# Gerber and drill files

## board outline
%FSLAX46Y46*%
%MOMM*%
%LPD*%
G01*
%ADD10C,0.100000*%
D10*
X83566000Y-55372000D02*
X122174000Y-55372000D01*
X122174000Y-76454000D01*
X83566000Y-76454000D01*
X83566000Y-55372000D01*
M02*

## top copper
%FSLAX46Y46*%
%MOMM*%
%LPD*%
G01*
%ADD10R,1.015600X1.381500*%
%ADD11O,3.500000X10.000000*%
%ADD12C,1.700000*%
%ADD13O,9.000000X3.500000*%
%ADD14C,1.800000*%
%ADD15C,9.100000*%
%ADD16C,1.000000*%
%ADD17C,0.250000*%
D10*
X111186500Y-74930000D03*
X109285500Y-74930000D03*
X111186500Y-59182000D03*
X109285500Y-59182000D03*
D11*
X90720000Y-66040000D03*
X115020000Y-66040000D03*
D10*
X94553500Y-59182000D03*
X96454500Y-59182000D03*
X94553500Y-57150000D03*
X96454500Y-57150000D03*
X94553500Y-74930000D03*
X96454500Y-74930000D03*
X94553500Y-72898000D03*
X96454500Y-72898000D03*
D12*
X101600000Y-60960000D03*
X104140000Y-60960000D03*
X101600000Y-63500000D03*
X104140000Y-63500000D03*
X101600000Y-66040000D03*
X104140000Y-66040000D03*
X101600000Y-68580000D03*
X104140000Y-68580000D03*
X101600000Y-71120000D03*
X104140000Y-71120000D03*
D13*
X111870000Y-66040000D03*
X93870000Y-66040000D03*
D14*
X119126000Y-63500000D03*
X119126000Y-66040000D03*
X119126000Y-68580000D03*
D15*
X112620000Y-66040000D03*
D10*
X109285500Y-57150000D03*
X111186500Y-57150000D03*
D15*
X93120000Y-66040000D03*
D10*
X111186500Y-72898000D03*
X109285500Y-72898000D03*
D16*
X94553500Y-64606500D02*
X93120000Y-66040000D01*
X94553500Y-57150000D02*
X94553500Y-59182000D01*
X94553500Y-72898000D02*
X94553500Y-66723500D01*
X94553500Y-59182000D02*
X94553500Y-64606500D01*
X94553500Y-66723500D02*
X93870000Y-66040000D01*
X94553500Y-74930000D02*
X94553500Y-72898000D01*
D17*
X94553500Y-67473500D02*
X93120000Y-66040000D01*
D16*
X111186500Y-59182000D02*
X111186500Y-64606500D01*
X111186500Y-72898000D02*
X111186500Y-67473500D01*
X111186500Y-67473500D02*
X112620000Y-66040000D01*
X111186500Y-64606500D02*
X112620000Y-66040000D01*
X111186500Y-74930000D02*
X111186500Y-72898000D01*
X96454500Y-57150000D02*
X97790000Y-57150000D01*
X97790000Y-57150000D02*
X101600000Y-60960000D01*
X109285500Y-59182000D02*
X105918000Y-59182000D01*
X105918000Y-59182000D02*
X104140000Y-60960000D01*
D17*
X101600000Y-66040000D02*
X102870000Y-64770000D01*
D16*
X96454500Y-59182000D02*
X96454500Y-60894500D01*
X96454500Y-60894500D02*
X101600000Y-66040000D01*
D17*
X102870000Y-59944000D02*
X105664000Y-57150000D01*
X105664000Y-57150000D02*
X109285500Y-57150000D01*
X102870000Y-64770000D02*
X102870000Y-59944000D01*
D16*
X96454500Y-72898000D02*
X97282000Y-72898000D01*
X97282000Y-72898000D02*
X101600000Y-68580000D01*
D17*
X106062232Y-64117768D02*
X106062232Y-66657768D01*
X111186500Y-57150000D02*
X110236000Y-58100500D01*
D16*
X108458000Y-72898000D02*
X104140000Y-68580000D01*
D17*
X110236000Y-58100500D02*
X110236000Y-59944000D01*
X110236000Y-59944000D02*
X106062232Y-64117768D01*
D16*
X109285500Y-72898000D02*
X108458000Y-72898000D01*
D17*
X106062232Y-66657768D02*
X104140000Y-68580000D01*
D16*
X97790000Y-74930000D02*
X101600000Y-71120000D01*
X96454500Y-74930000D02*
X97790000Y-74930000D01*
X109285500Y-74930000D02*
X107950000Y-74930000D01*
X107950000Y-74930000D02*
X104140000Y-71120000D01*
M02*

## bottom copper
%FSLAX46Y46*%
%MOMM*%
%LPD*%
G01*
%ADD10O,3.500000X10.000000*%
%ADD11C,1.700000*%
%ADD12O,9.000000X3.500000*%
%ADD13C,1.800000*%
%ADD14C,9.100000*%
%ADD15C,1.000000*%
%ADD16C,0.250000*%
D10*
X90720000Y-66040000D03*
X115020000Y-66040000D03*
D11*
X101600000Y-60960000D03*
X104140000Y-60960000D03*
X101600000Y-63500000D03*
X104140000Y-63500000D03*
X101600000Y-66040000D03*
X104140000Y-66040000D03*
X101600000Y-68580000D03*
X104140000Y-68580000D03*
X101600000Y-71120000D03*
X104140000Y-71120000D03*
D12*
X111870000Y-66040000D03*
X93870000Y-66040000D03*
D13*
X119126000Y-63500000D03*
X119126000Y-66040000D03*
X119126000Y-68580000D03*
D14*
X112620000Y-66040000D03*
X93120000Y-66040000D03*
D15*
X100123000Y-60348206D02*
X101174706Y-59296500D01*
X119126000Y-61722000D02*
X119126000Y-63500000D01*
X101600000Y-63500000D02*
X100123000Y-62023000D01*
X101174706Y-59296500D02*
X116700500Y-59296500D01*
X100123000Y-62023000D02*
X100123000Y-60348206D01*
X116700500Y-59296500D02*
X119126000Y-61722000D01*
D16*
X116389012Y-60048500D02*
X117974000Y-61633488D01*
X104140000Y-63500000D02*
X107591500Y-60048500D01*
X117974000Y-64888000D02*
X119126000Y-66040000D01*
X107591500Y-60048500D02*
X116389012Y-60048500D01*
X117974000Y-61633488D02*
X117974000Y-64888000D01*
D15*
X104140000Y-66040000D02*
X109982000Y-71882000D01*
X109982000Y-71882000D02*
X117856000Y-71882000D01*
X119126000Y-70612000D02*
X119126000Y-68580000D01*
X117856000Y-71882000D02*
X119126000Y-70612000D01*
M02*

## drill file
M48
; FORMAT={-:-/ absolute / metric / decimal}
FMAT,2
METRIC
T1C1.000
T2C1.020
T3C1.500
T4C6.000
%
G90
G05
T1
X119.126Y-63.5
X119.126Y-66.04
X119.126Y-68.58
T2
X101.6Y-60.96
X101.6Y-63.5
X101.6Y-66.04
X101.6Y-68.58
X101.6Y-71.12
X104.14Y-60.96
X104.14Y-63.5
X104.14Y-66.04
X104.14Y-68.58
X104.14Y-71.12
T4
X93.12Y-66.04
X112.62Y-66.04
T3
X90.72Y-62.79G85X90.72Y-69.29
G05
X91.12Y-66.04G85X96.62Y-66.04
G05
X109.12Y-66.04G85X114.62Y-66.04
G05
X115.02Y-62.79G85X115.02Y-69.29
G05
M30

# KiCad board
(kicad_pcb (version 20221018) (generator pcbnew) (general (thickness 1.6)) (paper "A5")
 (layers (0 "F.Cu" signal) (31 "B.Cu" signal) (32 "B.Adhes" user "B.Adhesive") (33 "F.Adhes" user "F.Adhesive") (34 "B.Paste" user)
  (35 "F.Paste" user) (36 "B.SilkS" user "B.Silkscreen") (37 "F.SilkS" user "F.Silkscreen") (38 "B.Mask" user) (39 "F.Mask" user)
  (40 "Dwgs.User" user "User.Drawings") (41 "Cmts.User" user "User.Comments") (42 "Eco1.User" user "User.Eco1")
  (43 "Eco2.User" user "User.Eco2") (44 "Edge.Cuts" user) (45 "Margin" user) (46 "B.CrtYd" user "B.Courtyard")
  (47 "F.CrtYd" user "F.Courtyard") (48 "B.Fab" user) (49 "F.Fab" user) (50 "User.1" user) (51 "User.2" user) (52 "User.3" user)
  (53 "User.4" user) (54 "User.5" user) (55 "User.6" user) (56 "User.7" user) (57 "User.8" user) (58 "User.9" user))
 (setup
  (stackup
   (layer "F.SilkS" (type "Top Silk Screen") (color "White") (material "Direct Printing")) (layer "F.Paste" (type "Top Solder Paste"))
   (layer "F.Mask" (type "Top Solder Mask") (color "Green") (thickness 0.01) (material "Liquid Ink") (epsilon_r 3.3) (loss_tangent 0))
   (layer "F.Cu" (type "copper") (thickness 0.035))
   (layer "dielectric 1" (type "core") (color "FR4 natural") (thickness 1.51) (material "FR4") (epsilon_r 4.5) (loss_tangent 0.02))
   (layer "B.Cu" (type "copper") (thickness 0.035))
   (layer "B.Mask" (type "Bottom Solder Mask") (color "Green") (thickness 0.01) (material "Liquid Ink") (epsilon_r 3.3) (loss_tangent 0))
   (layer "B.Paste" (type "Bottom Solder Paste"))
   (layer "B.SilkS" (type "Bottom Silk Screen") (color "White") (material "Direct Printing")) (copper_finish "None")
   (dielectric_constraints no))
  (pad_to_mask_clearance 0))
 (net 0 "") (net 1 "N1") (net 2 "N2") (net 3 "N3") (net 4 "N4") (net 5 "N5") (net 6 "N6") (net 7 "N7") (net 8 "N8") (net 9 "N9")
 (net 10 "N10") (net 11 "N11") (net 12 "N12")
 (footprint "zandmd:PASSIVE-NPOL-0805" (layer "F.Cu") (at 110.236 74.93 180)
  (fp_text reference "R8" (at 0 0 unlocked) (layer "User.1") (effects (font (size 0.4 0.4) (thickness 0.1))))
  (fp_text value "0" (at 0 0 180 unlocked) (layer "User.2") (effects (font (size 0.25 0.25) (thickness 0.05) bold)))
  (pad "1" smd rect (at -0.9505 0 180) (size 1.0156 1.3815) (layers "F.Cu" "F.Paste" "F.Mask") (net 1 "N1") (thermal_bridge_angle 45))
  (pad "2" smd rect (at 0.9505 0 180) (size 1.0156 1.3815) (layers "F.Cu" "F.Paste" "F.Mask") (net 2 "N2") (thermal_bridge_angle 45)))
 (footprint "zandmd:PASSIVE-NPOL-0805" (layer "F.Cu") (at 110.236 59.182 180)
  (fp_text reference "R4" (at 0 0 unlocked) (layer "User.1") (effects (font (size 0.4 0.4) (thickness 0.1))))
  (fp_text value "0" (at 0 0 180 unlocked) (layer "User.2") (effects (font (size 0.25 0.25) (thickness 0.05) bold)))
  (pad "1" smd rect (at -0.9505 0 180) (size 1.0156 1.3815) (layers "F.Cu" "F.Paste" "F.Mask") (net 1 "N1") (thermal_bridge_angle 45))
  (pad "2" smd rect (at 0.9505 0 180) (size 1.0156 1.3815) (layers "F.Cu" "F.Paste" "F.Mask") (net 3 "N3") (thermal_bridge_angle 45)))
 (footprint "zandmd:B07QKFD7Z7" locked (layer "F.Cu") (at 102.87 66.04) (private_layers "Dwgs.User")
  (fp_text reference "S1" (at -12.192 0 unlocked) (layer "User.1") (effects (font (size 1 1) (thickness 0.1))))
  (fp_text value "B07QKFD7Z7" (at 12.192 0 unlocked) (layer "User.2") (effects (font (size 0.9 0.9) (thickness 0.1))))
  (pad "1" thru_hole oval locked (at -12.15 0) (size 3.5 10) (drill oval 1.5 8) (layers "*.Cu" "*.Mask") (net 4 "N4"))
  (pad "2" thru_hole oval locked (at 12.15 0) (size 3.5 10) (drill oval 1.5 8) (layers "*.Cu" "*.Mask") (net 1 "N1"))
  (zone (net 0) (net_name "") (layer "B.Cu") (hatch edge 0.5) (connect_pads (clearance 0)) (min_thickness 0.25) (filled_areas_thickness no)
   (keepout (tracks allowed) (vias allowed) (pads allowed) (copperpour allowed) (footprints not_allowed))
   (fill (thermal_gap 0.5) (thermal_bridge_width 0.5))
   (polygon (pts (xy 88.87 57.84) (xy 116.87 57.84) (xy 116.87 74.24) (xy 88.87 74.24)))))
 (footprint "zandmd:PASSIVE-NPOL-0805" (layer "F.Cu") (at 95.504 59.182)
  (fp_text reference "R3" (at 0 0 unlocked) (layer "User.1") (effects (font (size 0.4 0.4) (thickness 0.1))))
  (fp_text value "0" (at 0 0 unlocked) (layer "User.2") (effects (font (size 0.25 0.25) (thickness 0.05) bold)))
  (pad "1" smd rect (at -0.9505 0) (size 1.0156 1.3815) (layers "F.Cu" "F.Paste" "F.Mask") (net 4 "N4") (thermal_bridge_angle 45))
  (pad "2" smd rect (at 0.9505 0) (size 1.0156 1.3815) (layers "F.Cu" "F.Paste" "F.Mask") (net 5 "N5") (thermal_bridge_angle 45)))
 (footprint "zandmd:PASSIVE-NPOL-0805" (layer "F.Cu") (at 95.504 57.15)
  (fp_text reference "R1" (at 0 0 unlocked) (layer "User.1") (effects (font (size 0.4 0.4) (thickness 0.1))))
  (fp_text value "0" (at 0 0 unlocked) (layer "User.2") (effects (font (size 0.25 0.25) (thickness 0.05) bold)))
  (pad "1" smd rect (at -0.9505 0) (size 1.0156 1.3815) (layers "F.Cu" "F.Paste" "F.Mask") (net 4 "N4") (thermal_bridge_angle 45))
  (pad "2" smd rect (at 0.9505 0) (size 1.0156 1.3815) (layers "F.Cu" "F.Paste" "F.Mask") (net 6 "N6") (thermal_bridge_angle 45)))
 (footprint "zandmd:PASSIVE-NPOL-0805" (layer "F.Cu") (at 95.504 74.93)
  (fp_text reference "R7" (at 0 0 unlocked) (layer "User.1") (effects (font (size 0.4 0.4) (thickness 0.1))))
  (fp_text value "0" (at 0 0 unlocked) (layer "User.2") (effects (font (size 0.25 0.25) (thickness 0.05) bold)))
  (pad "1" smd rect (at -0.9505 0) (size 1.0156 1.3815) (layers "F.Cu" "F.Paste" "F.Mask") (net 4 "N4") (thermal_bridge_angle 45))
  (pad "2" smd rect (at 0.9505 0) (size 1.0156 1.3815) (layers "F.Cu" "F.Paste" "F.Mask") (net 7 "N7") (thermal_bridge_angle 45)))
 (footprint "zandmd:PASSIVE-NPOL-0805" (layer "F.Cu") (at 95.504 72.898)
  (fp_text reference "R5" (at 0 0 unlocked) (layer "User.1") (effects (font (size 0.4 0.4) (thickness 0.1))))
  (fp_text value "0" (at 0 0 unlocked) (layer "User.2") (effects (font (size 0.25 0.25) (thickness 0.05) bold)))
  (pad "1" smd rect (at -0.9505 0) (size 1.0156 1.3815) (layers "F.Cu" "F.Paste" "F.Mask") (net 4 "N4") (thermal_bridge_angle 45))
  (pad "2" smd rect (at 0.9505 0) (size 1.0156 1.3815) (layers "F.Cu" "F.Paste" "F.Mask") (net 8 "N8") (thermal_bridge_angle 45)))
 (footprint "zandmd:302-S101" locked (layer "F.Cu") (at 102.87 66.04 -90)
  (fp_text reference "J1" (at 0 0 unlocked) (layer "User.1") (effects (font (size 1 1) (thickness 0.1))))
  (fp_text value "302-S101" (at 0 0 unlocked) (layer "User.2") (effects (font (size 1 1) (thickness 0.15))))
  (pad "1" thru_hole circle locked (at -5.08 1.27 270) (size 1.7 1.7) (drill 1.02) (layers "*.Cu" "*.Mask") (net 6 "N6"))
  (pad "2" thru_hole circle locked (at -5.08 -1.27 270) (size 1.7 1.7) (drill 1.02) (layers "*.Cu" "*.Mask") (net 3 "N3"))
  (pad "3" thru_hole circle locked (at -2.54 1.27 270) (size 1.7 1.7) (drill 1.02) (layers "*.Cu" "*.Mask") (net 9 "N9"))
  (pad "4" thru_hole circle locked (at -2.54 -1.27 270) (size 1.7 1.7) (drill 1.02) (layers "*.Cu" "*.Mask") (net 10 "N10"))
  (pad "5" thru_hole circle locked (at 0 1.27 270) (size 1.7 1.7) (drill 1.02) (layers "*.Cu" "*.Mask") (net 5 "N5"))
  (pad "6" thru_hole circle locked (at 0 -1.27 270) (size 1.7 1.7) (drill 1.02) (layers "*.Cu" "*.Mask") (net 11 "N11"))
  (pad "7" thru_hole circle locked (at 2.54 1.27 270) (size 1.7 1.7) (drill 1.02) (layers "*.Cu" "*.Mask") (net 8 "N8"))
  (pad "8" thru_hole circle locked (at 2.54 -1.27 270) (size 1.7 1.7) (drill 1.02) (layers "*.Cu" "*.Mask") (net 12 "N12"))
  (pad "9" thru_hole circle locked (at 5.08 1.27 270) (size 1.7 1.7) (drill 1.02) (layers "*.Cu" "*.Mask") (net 7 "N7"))
  (pad "10" thru_hole circle locked (at 5.08 -1.27 270) (size 1.7 1.7) (drill 1.02) (layers "*.Cu" "*.Mask") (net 2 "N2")))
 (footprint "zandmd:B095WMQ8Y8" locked (layer "F.Cu") (at 102.87 66.04) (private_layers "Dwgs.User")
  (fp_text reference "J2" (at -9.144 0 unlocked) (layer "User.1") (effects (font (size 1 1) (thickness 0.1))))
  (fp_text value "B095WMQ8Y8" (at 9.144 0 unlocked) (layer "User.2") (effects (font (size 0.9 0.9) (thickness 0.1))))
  (pad "1" thru_hole oval locked (at 9 0) (size 9 3.5) (drill oval 7 1.5) (layers "*.Cu" "*.Mask") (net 1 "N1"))
  (pad "2" thru_hole oval locked (at -9 0) (size 9 3.5) (drill oval 7 1.5) (layers "*.Cu" "*.Mask") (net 4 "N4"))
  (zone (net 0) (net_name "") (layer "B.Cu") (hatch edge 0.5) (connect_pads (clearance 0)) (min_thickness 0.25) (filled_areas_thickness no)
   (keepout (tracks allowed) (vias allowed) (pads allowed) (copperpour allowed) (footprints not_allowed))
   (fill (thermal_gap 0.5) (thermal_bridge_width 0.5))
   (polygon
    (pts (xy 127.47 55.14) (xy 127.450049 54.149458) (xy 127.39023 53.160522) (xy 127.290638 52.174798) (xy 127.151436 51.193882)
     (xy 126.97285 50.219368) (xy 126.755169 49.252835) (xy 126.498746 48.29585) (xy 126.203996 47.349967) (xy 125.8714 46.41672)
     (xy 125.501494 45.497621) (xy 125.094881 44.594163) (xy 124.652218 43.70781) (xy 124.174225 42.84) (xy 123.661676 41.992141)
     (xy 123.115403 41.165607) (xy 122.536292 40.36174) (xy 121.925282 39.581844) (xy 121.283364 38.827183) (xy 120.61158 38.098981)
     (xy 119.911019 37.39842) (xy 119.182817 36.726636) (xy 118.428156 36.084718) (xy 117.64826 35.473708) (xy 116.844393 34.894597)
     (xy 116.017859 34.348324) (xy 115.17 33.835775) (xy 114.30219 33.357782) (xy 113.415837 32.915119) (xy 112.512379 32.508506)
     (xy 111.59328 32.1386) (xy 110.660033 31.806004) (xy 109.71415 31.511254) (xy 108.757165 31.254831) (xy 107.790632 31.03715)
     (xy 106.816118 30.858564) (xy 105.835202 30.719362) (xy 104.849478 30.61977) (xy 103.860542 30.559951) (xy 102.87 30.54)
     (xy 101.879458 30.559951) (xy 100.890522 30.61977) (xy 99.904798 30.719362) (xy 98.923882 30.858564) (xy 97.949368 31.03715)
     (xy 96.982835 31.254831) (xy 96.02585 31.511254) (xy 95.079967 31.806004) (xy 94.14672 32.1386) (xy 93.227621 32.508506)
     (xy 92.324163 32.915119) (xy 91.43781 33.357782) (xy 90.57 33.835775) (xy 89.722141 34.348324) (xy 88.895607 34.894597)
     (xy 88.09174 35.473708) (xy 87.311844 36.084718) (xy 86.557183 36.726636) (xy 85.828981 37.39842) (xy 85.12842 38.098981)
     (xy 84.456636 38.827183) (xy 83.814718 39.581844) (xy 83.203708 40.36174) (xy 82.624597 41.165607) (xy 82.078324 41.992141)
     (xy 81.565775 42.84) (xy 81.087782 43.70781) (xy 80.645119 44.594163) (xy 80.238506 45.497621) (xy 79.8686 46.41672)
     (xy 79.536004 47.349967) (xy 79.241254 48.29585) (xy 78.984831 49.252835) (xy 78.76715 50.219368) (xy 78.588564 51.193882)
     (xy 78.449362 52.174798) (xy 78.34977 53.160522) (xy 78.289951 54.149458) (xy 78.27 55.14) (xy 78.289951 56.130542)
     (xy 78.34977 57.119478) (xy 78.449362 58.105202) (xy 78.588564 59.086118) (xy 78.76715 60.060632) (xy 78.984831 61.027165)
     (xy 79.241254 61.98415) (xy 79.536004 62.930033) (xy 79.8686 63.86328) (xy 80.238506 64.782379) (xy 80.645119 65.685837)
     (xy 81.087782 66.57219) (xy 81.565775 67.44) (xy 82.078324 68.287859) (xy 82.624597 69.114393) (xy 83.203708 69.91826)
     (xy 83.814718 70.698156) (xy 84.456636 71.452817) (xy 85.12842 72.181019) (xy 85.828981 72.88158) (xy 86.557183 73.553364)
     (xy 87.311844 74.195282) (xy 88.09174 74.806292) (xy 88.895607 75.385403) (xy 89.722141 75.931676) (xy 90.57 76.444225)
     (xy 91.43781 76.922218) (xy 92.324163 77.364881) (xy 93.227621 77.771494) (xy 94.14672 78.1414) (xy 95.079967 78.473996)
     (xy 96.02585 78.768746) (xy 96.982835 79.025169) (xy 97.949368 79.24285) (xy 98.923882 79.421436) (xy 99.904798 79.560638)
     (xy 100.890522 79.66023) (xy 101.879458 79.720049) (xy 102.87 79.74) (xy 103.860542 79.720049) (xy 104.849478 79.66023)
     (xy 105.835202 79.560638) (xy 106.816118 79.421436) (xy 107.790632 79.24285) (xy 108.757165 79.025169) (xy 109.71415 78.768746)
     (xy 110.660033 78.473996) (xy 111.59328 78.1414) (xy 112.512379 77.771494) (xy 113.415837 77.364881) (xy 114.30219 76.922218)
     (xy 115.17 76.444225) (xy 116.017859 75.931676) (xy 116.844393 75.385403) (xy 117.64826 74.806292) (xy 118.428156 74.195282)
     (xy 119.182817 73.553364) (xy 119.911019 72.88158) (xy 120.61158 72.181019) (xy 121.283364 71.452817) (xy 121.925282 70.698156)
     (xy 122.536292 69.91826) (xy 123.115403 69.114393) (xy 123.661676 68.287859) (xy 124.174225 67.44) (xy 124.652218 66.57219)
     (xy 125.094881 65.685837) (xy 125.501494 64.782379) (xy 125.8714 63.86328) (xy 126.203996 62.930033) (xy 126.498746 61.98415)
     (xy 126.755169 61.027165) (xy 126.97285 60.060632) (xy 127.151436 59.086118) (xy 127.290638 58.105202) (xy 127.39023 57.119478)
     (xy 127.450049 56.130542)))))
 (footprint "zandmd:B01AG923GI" (layer "F.Cu") (at 119.126 66.04 -90)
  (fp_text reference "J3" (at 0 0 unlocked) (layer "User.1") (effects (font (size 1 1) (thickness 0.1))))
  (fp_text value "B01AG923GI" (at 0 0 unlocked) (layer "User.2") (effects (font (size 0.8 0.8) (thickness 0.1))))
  (pad "1" thru_hole circle (at -2.54 0 270) (size 1.8 1.8) (drill 1) (layers "*.Cu" "*.Mask") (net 9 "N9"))
  (pad "2" thru_hole circle (at 0 0 270) (size 1.8 1.8) (drill 1) (layers "*.Cu" "*.Mask") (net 10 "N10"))
  (pad "3" thru_hole circle (at 2.54 0 270) (size 1.8 1.8) (drill 1) (layers "*.Cu" "*.Mask") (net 11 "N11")))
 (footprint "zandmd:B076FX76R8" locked (layer "F.Cu") (at 112.62 66.04 180) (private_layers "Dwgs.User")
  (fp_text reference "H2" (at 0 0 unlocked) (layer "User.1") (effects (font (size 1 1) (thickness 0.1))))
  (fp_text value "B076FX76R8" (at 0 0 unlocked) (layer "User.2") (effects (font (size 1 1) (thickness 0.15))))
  (pad "1" thru_hole circle locked (at 0 0 180) (size 9.1 9.1) (drill 6) (layers "*.Cu" "*.Mask") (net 1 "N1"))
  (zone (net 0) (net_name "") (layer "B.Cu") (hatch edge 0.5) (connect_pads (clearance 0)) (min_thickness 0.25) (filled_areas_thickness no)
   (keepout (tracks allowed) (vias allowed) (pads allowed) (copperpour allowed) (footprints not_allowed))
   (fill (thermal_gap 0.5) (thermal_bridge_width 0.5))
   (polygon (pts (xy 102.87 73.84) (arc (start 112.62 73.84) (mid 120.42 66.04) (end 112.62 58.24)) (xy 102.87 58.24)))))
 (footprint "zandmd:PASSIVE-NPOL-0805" (layer "F.Cu") (at 110.236 57.15)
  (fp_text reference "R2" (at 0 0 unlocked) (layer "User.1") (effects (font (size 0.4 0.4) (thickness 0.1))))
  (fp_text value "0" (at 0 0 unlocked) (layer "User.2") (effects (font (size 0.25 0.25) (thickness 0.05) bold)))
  (pad "1" smd rect (at -0.9505 0) (size 1.0156 1.3815) (layers "F.Cu" "F.Paste" "F.Mask") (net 5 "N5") (thermal_bridge_angle 45))
  (pad "2" smd rect (at 0.9505 0) (size 1.0156 1.3815) (layers "F.Cu" "F.Paste" "F.Mask") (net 12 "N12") (thermal_bridge_angle 45)))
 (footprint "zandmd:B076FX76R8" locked (layer "F.Cu") (at 93.12 66.04) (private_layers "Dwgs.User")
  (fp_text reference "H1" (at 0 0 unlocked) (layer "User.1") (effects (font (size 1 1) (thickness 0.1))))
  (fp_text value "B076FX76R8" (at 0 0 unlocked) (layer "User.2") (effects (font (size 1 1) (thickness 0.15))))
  (pad "1" thru_hole circle locked (at 0 0) (size 9.1 9.1) (drill 6) (layers "*.Cu" "*.Mask") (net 4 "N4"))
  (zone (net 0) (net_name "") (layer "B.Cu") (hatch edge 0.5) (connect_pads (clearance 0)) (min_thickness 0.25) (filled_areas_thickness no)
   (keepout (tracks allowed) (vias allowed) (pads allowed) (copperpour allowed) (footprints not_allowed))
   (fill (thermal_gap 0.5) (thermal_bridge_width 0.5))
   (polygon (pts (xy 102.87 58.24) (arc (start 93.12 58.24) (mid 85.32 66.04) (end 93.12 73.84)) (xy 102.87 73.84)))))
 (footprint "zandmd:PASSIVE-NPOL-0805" (layer "F.Cu") (at 110.236 72.898 180)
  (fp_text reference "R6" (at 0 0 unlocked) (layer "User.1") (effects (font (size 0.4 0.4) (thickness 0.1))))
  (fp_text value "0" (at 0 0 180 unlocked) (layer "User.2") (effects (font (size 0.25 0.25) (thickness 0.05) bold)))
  (pad "1" smd rect (at -0.9505 0 180) (size 1.0156 1.3815) (layers "F.Cu" "F.Paste" "F.Mask") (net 1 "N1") (thermal_bridge_angle 45))
  (pad "2" smd rect (at 0.9505 0 180) (size 1.0156 1.3815) (layers "F.Cu" "F.Paste" "F.Mask") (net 12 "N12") (thermal_bridge_angle 45)))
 (gr_rect (start 83.566 55.372) (end 122.174 76.454) (stroke (width 0.1) (type default)) (fill none) (layer "Edge.Cuts"))
 (segment (start 94.5535 64.6065) (end 93.12 66.04) (width 1) (layer "F.Cu") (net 4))
 (segment (start 94.5535 57.15) (end 94.5535 59.182) (width 1) (layer "F.Cu") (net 4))
 (segment (start 94.5535 72.898) (end 94.5535 66.7235) (width 1) (layer "F.Cu") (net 4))
 (segment (start 94.5535 59.182) (end 94.5535 64.6065) (width 1) (layer "F.Cu") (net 4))
 (segment (start 94.5535 66.7235) (end 93.87 66.04) (width 1) (layer "F.Cu") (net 4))
 (segment (start 94.5535 74.93) (end 94.5535 72.898) (width 1) (layer "F.Cu") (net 4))
 (segment (start 94.5535 67.4735) (end 93.12 66.04) (width 0.25) (layer "F.Cu") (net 4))
 (segment (start 111.1865 59.182) (end 111.1865 64.6065) (width 1) (layer "F.Cu") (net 1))
 (segment (start 111.1865 72.898) (end 111.1865 67.4735) (width 1) (layer "F.Cu") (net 1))
 (segment (start 111.1865 67.4735) (end 112.62 66.04) (width 1) (layer "F.Cu") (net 1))
 (segment (start 111.1865 64.6065) (end 112.62 66.04) (width 1) (layer "F.Cu") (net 1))
 (segment (start 111.1865 74.93) (end 111.1865 72.898) (width 1) (layer "F.Cu") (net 1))
 (segment (start 96.4545 57.15) (end 97.79 57.15) (width 1) (layer "F.Cu") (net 6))
 (segment (start 97.79 57.15) (end 101.6 60.96) (width 1) (layer "F.Cu") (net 6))
 (segment (start 109.2855 59.182) (end 105.918 59.182) (width 1) (layer "F.Cu") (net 3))
 (segment (start 105.918 59.182) (end 104.14 60.96) (width 1) (layer "F.Cu") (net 3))
 (segment (start 100.123 60.348206) (end 101.174706 59.2965) (width 1) (layer "B.Cu") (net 9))
 (segment (start 119.126 61.722) (end 119.126 63.5) (width 1) (layer "B.Cu") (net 9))
 (segment (start 101.6 63.5) (end 100.123 62.023) (width 1) (layer "B.Cu") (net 9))
 (segment (start 101.174706 59.2965) (end 116.7005 59.2965) (width 1) (layer "B.Cu") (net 9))
 (segment (start 100.123 62.023) (end 100.123 60.348206) (width 1) (layer "B.Cu") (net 9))
 (segment (start 116.7005 59.2965) (end 119.126 61.722) (width 1) (layer "B.Cu") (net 9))
 (segment (start 116.389012 60.0485) (end 117.974 61.633488) (width 0.25) (layer "B.Cu") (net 10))
 (segment (start 104.14 63.5) (end 107.5915 60.0485) (width 0.25) (layer "B.Cu") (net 10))
 (segment (start 117.974 64.888) (end 119.126 66.04) (width 0.25) (layer "B.Cu") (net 10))
 (segment (start 107.5915 60.0485) (end 116.389012 60.0485) (width 0.25) (layer "B.Cu") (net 10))
 (segment (start 117.974 61.633488) (end 117.974 64.888) (width 0.25) (layer "B.Cu") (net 10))
 (segment (start 101.6 66.04) (end 102.87 64.77) (width 0.25) (layer "F.Cu") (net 5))
 (segment (start 96.4545 59.182) (end 96.4545 60.8945) (width 1) (layer "F.Cu") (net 5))
 (segment (start 96.4545 60.8945) (end 101.6 66.04) (width 1) (layer "F.Cu") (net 5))
 (segment (start 102.87 59.944) (end 105.664 57.15) (width 0.25) (layer "F.Cu") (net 5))
 (segment (start 105.664 57.15) (end 109.2855 57.15) (width 0.25) (layer "F.Cu") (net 5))
 (segment (start 102.87 64.77) (end 102.87 59.944) (width 0.25) (layer "F.Cu") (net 5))
 (segment (start 104.14 66.04) (end 109.982 71.882) (width 1) (layer "B.Cu") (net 11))
 (segment (start 109.982 71.882) (end 117.856 71.882) (width 1) (layer "B.Cu") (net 11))
 (segment (start 119.126 70.612) (end 119.126 68.58) (width 1) (layer "B.Cu") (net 11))
 (segment (start 117.856 71.882) (end 119.126 70.612) (width 1) (layer "B.Cu") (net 11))
 (segment (start 96.4545 72.898) (end 97.282 72.898) (width 1) (layer "F.Cu") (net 8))
 (segment (start 97.282 72.898) (end 101.6 68.58) (width 1) (layer "F.Cu") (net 8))
 (segment (start 106.062232 64.117768) (end 106.062232 66.657768) (width 0.25) (layer "F.Cu") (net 12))
 (segment (start 111.1865 57.15) (end 110.236 58.1005) (width 0.25) (layer "F.Cu") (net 12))
 (segment (start 108.458 72.898) (end 104.14 68.58) (width 1) (layer "F.Cu") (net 12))
 (segment (start 110.236 58.1005) (end 110.236 59.944) (width 0.25) (layer "F.Cu") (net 12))
 (segment (start 110.236 59.944) (end 106.062232 64.117768) (width 0.25) (layer "F.Cu") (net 12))
 (segment (start 109.2855 72.898) (end 108.458 72.898) (width 1) (layer "F.Cu") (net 12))
 (segment (start 106.062232 66.657768) (end 104.14 68.58) (width 0.25) (layer "F.Cu") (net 12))
 (segment (start 97.79 74.93) (end 101.6 71.12) (width 1) (layer "F.Cu") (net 7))
 (segment (start 96.4545 74.93) (end 97.79 74.93) (width 1) (layer "F.Cu") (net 7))
 (segment (start 109.2855 74.93) (end 107.95 74.93) (width 1) (layer "F.Cu") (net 2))
 (segment (start 107.95 74.93) (end 104.14 71.12) (width 1) (layer "F.Cu") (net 2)))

